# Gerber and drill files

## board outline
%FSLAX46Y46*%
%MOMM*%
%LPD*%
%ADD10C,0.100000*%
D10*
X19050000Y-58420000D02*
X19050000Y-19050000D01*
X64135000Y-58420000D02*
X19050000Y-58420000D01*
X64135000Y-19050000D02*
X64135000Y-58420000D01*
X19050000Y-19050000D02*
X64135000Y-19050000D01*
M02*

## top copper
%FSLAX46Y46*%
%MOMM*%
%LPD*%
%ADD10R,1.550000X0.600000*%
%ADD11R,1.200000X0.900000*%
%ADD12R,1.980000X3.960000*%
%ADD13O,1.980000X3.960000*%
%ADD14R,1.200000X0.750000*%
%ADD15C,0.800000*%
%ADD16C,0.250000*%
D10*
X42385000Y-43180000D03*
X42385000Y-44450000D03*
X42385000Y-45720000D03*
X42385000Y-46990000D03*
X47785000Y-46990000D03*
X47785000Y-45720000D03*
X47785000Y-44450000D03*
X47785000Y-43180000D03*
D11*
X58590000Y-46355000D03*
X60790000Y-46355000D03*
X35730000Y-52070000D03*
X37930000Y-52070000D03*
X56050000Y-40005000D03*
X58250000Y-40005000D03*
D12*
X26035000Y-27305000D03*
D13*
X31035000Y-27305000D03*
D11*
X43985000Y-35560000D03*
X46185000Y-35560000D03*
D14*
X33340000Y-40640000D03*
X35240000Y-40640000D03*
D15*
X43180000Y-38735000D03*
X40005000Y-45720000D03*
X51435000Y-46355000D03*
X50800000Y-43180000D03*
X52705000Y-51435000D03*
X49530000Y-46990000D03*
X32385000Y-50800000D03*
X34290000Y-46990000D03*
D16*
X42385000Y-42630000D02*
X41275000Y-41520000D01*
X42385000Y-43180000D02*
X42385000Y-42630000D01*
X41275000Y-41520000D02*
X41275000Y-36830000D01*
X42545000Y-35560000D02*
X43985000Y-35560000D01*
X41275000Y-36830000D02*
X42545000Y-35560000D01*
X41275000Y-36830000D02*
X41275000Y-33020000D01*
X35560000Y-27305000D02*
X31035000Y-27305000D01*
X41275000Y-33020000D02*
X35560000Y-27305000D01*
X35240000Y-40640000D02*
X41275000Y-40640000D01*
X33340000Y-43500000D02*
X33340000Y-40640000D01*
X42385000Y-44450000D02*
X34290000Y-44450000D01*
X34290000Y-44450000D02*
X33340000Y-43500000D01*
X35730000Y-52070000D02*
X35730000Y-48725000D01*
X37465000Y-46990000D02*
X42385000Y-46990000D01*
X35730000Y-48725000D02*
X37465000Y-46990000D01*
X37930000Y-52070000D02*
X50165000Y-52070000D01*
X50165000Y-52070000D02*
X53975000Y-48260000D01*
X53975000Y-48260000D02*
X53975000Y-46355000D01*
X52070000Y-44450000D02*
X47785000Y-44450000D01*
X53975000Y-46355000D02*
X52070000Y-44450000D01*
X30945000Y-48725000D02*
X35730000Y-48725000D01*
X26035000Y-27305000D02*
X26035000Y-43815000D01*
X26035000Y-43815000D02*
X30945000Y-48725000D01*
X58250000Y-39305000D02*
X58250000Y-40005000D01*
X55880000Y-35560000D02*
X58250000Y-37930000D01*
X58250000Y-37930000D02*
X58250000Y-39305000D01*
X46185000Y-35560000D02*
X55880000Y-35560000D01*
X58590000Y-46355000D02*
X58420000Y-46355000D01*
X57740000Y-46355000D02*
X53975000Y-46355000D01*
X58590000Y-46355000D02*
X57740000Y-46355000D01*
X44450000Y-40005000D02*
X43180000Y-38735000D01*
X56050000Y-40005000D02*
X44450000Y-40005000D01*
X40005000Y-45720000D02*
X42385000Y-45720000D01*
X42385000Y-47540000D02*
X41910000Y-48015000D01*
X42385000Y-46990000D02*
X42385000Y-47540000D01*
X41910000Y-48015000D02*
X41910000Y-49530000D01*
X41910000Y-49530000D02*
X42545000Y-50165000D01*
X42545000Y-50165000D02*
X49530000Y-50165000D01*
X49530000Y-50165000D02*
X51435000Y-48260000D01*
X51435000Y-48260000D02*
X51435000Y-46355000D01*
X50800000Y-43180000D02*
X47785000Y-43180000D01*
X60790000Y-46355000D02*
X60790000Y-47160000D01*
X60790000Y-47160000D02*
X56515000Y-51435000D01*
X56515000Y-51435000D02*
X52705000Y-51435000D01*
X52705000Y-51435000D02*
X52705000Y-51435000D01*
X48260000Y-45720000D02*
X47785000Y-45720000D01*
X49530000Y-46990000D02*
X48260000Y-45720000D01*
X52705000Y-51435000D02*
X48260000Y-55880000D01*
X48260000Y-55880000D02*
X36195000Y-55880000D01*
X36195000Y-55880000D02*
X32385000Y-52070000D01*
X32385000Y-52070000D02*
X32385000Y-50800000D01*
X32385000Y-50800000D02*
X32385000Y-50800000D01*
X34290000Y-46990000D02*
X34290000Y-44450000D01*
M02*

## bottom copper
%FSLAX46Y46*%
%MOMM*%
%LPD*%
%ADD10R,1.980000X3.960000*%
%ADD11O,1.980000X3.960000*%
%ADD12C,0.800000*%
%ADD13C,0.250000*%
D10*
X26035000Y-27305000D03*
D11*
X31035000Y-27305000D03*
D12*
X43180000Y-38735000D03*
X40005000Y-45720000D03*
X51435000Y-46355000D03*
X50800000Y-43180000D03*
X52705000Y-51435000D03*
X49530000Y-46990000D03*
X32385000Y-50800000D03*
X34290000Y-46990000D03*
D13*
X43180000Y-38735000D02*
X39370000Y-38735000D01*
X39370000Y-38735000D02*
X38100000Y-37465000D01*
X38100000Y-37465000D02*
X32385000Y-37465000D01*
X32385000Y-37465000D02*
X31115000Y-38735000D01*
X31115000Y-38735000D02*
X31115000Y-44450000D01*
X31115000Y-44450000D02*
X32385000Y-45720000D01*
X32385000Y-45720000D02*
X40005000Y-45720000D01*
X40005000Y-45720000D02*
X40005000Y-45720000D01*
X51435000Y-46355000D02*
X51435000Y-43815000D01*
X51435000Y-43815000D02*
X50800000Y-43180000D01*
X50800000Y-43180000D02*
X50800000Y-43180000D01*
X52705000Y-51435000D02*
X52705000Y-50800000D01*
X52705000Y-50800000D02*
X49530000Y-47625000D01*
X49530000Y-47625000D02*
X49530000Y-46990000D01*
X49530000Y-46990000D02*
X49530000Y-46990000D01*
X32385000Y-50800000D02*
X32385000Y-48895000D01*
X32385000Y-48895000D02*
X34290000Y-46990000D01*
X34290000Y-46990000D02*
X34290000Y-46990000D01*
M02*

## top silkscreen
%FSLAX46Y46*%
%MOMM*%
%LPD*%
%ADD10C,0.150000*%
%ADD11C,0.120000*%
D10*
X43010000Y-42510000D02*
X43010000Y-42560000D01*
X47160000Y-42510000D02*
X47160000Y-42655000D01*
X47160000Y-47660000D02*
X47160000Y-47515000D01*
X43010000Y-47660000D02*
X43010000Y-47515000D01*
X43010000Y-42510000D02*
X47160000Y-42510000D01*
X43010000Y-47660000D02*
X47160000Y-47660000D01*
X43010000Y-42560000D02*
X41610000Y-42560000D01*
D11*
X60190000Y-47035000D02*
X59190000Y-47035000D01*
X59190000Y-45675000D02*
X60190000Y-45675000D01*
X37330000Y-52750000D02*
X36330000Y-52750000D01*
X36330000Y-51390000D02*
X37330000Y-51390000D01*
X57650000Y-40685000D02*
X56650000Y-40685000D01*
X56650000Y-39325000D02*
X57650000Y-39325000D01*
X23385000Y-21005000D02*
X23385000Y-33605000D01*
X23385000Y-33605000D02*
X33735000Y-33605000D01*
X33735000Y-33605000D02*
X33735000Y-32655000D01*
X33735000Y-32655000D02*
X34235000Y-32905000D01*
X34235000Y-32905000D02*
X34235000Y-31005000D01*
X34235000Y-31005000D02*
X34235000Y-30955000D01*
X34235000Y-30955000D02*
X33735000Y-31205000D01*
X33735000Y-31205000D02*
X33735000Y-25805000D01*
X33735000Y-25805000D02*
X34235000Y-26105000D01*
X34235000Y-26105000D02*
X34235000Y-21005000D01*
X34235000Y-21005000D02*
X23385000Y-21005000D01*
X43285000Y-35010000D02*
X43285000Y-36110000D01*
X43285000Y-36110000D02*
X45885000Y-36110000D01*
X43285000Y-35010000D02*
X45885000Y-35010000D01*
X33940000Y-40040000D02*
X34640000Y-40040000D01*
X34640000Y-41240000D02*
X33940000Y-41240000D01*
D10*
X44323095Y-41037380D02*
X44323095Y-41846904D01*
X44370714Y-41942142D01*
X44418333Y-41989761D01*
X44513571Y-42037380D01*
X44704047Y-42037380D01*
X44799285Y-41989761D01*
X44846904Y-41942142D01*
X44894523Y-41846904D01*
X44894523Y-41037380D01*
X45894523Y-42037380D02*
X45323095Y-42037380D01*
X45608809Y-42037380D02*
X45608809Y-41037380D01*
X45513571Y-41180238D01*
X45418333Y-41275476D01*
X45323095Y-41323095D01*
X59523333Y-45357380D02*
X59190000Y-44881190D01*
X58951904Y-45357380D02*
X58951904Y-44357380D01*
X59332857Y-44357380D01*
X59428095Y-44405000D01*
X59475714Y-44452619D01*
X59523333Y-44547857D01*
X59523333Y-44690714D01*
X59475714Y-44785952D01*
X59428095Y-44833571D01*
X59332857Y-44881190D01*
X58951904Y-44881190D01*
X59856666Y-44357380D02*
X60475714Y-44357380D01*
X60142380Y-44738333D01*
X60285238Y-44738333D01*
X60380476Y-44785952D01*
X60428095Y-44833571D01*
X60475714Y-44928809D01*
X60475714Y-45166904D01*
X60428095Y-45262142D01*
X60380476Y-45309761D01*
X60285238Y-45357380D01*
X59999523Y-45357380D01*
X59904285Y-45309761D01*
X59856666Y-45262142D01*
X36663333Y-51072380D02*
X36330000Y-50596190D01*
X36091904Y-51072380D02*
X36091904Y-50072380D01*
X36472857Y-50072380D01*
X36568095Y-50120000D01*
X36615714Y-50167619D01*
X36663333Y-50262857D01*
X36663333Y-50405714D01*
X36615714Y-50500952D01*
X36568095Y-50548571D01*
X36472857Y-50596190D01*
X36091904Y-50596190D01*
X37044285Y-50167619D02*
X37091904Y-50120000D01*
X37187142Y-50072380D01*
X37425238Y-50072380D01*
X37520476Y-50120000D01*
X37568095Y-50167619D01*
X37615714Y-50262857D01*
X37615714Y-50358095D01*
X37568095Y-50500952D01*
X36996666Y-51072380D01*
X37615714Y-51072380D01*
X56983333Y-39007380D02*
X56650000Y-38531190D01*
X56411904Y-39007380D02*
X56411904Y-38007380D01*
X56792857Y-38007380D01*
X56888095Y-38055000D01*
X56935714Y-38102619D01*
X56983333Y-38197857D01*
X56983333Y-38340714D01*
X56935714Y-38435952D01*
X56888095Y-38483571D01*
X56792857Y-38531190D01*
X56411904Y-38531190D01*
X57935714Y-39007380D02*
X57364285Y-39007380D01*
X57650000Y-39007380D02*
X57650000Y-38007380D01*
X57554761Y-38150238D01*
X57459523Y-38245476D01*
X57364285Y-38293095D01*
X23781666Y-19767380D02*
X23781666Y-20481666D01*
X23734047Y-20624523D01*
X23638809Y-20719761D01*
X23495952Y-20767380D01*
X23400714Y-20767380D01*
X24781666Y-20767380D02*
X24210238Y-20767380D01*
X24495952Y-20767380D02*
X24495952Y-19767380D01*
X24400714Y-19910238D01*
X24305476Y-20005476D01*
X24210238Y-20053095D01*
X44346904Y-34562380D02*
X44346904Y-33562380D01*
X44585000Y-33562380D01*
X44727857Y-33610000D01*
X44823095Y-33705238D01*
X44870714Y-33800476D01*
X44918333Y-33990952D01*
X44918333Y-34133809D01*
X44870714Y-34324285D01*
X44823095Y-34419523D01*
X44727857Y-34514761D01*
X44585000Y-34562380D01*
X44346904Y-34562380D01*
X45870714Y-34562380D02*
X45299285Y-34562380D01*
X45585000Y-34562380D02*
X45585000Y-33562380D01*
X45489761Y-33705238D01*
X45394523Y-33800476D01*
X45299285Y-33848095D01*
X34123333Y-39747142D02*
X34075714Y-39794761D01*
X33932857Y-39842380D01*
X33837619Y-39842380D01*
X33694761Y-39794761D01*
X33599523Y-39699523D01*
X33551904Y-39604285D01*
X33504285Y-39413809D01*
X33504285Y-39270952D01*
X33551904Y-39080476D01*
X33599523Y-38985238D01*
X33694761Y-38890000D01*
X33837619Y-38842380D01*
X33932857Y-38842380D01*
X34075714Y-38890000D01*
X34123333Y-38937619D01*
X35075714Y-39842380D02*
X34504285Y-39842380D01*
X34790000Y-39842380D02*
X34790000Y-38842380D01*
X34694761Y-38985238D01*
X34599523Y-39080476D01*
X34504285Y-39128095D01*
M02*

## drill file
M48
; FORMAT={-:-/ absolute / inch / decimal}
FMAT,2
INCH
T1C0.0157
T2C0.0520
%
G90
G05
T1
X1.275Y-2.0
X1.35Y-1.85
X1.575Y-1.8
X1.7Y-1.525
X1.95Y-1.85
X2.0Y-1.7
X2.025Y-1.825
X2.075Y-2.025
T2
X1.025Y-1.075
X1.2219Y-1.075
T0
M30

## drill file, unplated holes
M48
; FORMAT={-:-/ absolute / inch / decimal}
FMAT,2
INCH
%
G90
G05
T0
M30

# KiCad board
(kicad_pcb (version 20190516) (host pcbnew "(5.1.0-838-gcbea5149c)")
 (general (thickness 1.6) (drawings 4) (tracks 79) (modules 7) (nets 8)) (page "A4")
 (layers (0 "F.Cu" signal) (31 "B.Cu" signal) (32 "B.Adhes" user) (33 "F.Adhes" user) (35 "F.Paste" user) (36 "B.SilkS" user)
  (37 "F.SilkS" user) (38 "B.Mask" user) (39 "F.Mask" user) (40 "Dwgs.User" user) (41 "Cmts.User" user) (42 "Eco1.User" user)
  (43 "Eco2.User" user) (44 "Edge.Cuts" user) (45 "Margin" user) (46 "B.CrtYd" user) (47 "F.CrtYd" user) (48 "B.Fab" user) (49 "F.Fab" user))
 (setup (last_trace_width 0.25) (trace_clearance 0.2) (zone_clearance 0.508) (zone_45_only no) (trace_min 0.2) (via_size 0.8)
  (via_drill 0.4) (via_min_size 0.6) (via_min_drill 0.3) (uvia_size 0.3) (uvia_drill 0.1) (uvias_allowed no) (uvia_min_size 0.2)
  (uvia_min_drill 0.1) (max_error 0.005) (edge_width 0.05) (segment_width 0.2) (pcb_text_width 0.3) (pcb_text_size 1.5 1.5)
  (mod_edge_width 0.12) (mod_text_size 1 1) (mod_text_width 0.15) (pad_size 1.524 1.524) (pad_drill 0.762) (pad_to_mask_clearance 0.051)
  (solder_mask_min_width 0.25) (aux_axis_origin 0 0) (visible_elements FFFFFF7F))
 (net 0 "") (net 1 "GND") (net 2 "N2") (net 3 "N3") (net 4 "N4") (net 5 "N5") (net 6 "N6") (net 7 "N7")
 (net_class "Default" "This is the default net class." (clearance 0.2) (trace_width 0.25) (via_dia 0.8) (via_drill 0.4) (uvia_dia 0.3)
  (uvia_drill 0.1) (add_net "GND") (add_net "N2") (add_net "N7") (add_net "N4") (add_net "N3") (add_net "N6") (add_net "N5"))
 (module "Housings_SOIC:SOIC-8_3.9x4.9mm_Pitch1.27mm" (layer "F.Cu") (at 45.085 45.085)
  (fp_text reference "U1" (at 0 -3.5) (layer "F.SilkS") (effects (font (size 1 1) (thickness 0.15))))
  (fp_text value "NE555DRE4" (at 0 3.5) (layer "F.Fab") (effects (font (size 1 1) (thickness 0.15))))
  (fp_line (start -2.075 -2.575) (end -2.075 -2.525) (layer "F.SilkS") (width 0.15))
  (fp_line (start 2.075 -2.575) (end 2.075 -2.43) (layer "F.SilkS") (width 0.15))
  (fp_line (start 2.075 2.575) (end 2.075 2.43) (layer "F.SilkS") (width 0.15))
  (fp_line (start -2.075 2.575) (end -2.075 2.43) (layer "F.SilkS") (width 0.15))
  (fp_line (start -2.075 -2.575) (end 2.075 -2.575) (layer "F.SilkS") (width 0.15))
  (fp_line (start -2.075 2.575) (end 2.075 2.575) (layer "F.SilkS") (width 0.15))
  (fp_line (start -2.075 -2.525) (end -3.475 -2.525) (layer "F.SilkS") (width 0.15))
  (pad "1" smd rect (at -2.7 -1.905) (size 1.55 0.6) (layers "F.Cu" "F.Paste" "F.Mask") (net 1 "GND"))
  (pad "2" smd rect (at -2.7 -0.635) (size 1.55 0.6) (layers "F.Cu" "F.Paste" "F.Mask") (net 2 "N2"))
  (pad "3" smd rect (at -2.7 0.635) (size 1.55 0.6) (layers "F.Cu" "F.Paste" "F.Mask") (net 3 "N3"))
  (pad "4" smd rect (at -2.7 1.905) (size 1.55 0.6) (layers "F.Cu" "F.Paste" "F.Mask") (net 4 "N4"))
  (pad "5" smd rect (at 2.7 1.905) (size 1.55 0.6) (layers "F.Cu" "F.Paste" "F.Mask") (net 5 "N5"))
  (pad "6" smd rect (at 2.7 0.635) (size 1.55 0.6) (layers "F.Cu" "F.Paste" "F.Mask") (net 2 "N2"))
  (pad "7" smd rect (at 2.7 -0.635) (size 1.55 0.6) (layers "F.Cu" "F.Paste" "F.Mask") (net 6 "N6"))
  (pad "8" smd rect (at 2.7 -1.905) (size 1.55 0.6) (layers "F.Cu" "F.Paste" "F.Mask") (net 4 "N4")))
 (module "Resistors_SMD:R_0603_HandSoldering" (layer "F.Cu") (at 59.69 46.355)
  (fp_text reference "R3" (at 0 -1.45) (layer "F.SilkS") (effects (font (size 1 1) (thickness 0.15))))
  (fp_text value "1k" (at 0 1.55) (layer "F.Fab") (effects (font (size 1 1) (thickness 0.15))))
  (fp_line (start 0.5 0.68) (end -0.5 0.68) (layer "F.SilkS") (width 0.12))
  (fp_line (start -0.5 -0.68) (end 0.5 -0.68) (layer "F.SilkS") (width 0.12))
  (pad "1" smd rect (at -1.1 0) (size 1.2 0.9) (layers "F.Cu" "F.Paste" "F.Mask") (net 6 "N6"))
  (pad "2" smd rect (at 1.1 0) (size 1.2 0.9) (layers "F.Cu" "F.Paste" "F.Mask") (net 2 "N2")))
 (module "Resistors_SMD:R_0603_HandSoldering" (layer "F.Cu") (at 36.83 52.07)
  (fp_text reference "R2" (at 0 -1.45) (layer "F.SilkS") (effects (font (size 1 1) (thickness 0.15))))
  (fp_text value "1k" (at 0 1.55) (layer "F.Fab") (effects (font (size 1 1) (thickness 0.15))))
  (fp_line (start 0.5 0.68) (end -0.5 0.68) (layer "F.SilkS") (width 0.12))
  (fp_line (start -0.5 -0.68) (end 0.5 -0.68) (layer "F.SilkS") (width 0.12))
  (pad "1" smd rect (at -1.1 0) (size 1.2 0.9) (layers "F.Cu" "F.Paste" "F.Mask") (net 4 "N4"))
  (pad "2" smd rect (at 1.1 0) (size 1.2 0.9) (layers "F.Cu" "F.Paste" "F.Mask") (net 6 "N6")))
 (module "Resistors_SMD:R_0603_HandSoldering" (layer "F.Cu") (at 57.15 40.005)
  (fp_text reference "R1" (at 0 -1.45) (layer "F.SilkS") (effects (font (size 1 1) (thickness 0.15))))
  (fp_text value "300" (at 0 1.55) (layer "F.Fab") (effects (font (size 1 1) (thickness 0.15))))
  (fp_line (start 0.5 0.68) (end -0.5 0.68) (layer "F.SilkS") (width 0.12))
  (fp_line (start -0.5 -0.68) (end 0.5 -0.68) (layer "F.SilkS") (width 0.12))
  (pad "1" smd rect (at -1.1 0) (size 1.2 0.9) (layers "F.Cu" "F.Paste" "F.Mask") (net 3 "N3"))
  (pad "2" smd rect (at 1.1 0) (size 1.2 0.9) (layers "F.Cu" "F.Paste" "F.Mask") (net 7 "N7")))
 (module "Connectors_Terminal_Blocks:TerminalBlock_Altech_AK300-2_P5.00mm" (layer "F.Cu") (at 26.035 27.305)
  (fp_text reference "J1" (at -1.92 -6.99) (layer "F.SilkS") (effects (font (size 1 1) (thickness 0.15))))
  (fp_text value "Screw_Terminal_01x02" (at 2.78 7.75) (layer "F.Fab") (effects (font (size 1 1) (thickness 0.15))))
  (fp_line (start -2.65 -6.3) (end -2.65 6.3) (layer "F.SilkS") (width 0.12))
  (fp_line (start -2.65 6.3) (end 7.7 6.3) (layer "F.SilkS") (width 0.12))
  (fp_line (start 7.7 6.3) (end 7.7 5.35) (layer "F.SilkS") (width 0.12))
  (fp_line (start 7.7 5.35) (end 8.2 5.6) (layer "F.SilkS") (width 0.12))
  (fp_line (start 8.2 5.6) (end 8.2 3.7) (layer "F.SilkS") (width 0.12))
  (fp_line (start 8.2 3.7) (end 8.2 3.65) (layer "F.SilkS") (width 0.12))
  (fp_line (start 8.2 3.65) (end 7.7 3.9) (layer "F.SilkS") (width 0.12))
  (fp_line (start 7.7 3.9) (end 7.7 -1.5) (layer "F.SilkS") (width 0.12))
  (fp_line (start 7.7 -1.5) (end 8.2 -1.2) (layer "F.SilkS") (width 0.12))
  (fp_line (start 8.2 -1.2) (end 8.2 -6.3) (layer "F.SilkS") (width 0.12))
  (fp_line (start 8.2 -6.3) (end -2.65 -6.3) (layer "F.SilkS") (width 0.12))
  (pad "1" thru_hole rect (at 0 0) (size 1.98 3.96) (drill 1.32) (layers *.Cu *.Mask) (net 4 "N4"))
  (pad "2" thru_hole oval (at 5 0) (size 1.98 3.96) (drill 1.32) (layers *.Cu *.Mask) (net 1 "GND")))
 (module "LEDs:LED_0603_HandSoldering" (layer "F.Cu") (at 45.085 35.56)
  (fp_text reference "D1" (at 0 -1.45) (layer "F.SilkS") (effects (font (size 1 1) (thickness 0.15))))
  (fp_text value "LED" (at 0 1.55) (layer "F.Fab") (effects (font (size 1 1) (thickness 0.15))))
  (fp_line (start -1.8 -0.55) (end -1.8 0.55) (layer "F.SilkS") (width 0.12))
  (fp_line (start -1.8 0.55) (end 0.8 0.55) (layer "F.SilkS") (width 0.12))
  (fp_line (start -1.8 -0.55) (end 0.8 -0.55) (layer "F.SilkS") (width 0.12))
  (pad "1" smd rect (at -1.1 0) (size 1.2 0.9) (layers "F.Cu" "F.Paste" "F.Mask") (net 1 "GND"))
  (pad "2" smd rect (at 1.1 0) (size 1.2 0.9) (layers "F.Cu" "F.Paste" "F.Mask") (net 7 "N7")))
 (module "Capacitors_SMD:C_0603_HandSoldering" (layer "F.Cu") (at 34.29 40.64)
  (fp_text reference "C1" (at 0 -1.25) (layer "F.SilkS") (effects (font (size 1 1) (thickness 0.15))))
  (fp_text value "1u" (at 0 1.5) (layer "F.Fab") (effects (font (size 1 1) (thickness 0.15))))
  (fp_line (start -0.35 -0.6) (end 0.35 -0.6) (layer "F.SilkS") (width 0.12))
  (fp_line (start 0.35 0.6) (end -0.35 0.6) (layer "F.SilkS") (width 0.12))
  (pad "1" smd rect (at -0.95 0) (size 1.2 0.75) (layers "F.Cu" "F.Paste" "F.Mask") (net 2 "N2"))
  (pad "2" smd rect (at 0.95 0) (size 1.2 0.75) (layers "F.Cu" "F.Paste" "F.Mask") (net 1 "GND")))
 (gr_line (start 19.05 58.42) (end 19.05 19.05) (layer "Edge.Cuts") (width 0.1))
 (gr_line (start 64.135 58.42) (end 19.05 58.42) (layer "Edge.Cuts") (width 0.1))
 (gr_line (start 64.135 19.05) (end 64.135 58.42) (layer "Edge.Cuts") (width 0.1))
 (gr_line (start 19.05 19.05) (end 64.135 19.05) (layer "Edge.Cuts") (width 0.1))
 (segment (start 42.385 42.63) (end 41.275 41.52) (width 0.25) (layer "F.Cu") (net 1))
 (segment (start 42.385 43.18) (end 42.385 42.63) (width 0.25) (layer "F.Cu") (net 1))
 (segment (start 41.275 41.52) (end 41.275 36.83) (width 0.25) (layer "F.Cu") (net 1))
 (segment (start 42.545 35.56) (end 43.985 35.56) (width 0.25) (layer "F.Cu") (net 1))
 (segment (start 41.275 36.83) (end 42.545 35.56) (width 0.25) (layer "F.Cu") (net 1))
 (segment (start 41.275 36.83) (end 41.275 33.02) (width 0.25) (layer "F.Cu") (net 1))
 (segment (start 35.56 27.305) (end 31.035 27.305) (width 0.25) (layer "F.Cu") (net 1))
 (segment (start 41.275 33.02) (end 35.56 27.305) (width 0.25) (layer "F.Cu") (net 1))
 (segment (start 35.24 40.64) (end 41.275 40.64) (width 0.25) (layer "F.Cu") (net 1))
 (segment (start 33.34 43.5) (end 33.34 40.64) (width 0.25) (layer "F.Cu") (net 2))
 (segment (start 42.385 44.45) (end 34.29 44.45) (width 0.25) (layer "F.Cu") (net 2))
 (segment (start 34.29 44.45) (end 33.34 43.5) (width 0.25) (layer "F.Cu") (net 2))
 (segment (start 35.73 52.07) (end 35.73 48.725) (width 0.25) (layer "F.Cu") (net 4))
 (segment (start 37.465 46.99) (end 42.385 46.99) (width 0.25) (layer "F.Cu") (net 4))
 (segment (start 35.73 48.725) (end 37.465 46.99) (width 0.25) (layer "F.Cu") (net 4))
 (segment (start 37.93 52.07) (end 50.165 52.07) (width 0.25) (layer "F.Cu") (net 6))
 (segment (start 50.165 52.07) (end 53.975 48.26) (width 0.25) (layer "F.Cu") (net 6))
 (segment (start 53.975 48.26) (end 53.975 46.355) (width 0.25) (layer "F.Cu") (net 6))
 (segment (start 52.07 44.45) (end 47.785 44.45) (width 0.25) (layer "F.Cu") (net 6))
 (segment (start 53.975 46.355) (end 52.07 44.45) (width 0.25) (layer "F.Cu") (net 6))
 (segment (start 30.945 48.725) (end 35.73 48.725) (width 0.25) (layer "F.Cu") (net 4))
 (segment (start 26.035 27.305) (end 26.035 43.815) (width 0.25) (layer "F.Cu") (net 4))
 (segment (start 26.035 43.815) (end 30.945 48.725) (width 0.25) (layer "F.Cu") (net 4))
 (segment (start 58.25 39.305) (end 58.25 40.005) (width 0.25) (layer "F.Cu") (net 7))
 (segment (start 55.88 35.56) (end 58.25 37.93) (width 0.25) (layer "F.Cu") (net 7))
 (segment (start 58.25 37.93) (end 58.25 39.305) (width 0.25) (layer "F.Cu") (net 7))
 (segment (start 46.185 35.56) (end 55.88 35.56) (width 0.25) (layer "F.Cu") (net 7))
 (segment (start 58.59 46.355) (end 58.42 46.355) (width 0.25) (layer "F.Cu") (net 6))
 (segment (start 57.74 46.355) (end 53.975 46.355) (width 0.25) (layer "F.Cu") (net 6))
 (segment (start 58.59 46.355) (end 57.74 46.355) (width 0.25) (layer "F.Cu") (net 6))
 (via (at 43.18 38.735) (size 0.8) (drill 0.4) (layers "F.Cu" "B.Cu") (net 3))
 (segment (start 44.45 40.005) (end 43.18 38.735) (width 0.25) (layer "F.Cu") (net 3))
 (segment (start 56.05 40.005) (end 44.45 40.005) (width 0.25) (layer "F.Cu") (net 3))
 (segment (start 43.18 38.735) (end 39.37 38.735) (width 0.25) (layer "B.Cu") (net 3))
 (segment (start 39.37 38.735) (end 38.1 37.465) (width 0.25) (layer "B.Cu") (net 3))
 (segment (start 38.1 37.465) (end 32.385 37.465) (width 0.25) (layer "B.Cu") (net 3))
 (segment (start 32.385 37.465) (end 31.115 38.735) (width 0.25) (layer "B.Cu") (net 3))
 (segment (start 31.115 38.735) (end 31.115 44.45) (width 0.25) (layer "B.Cu") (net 3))
 (segment (start 31.115 44.45) (end 32.385 45.72) (width 0.25) (layer "B.Cu") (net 3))
 (segment (start 32.385 45.72) (end 40.005 45.72) (width 0.25) (layer "B.Cu") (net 3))
 (segment (start 40.005 45.72) (end 40.005 45.72) (width 0.25) (layer "B.Cu") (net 3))
 (via (at 40.005 45.72) (size 0.8) (drill 0.4) (layers "F.Cu" "B.Cu") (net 3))
 (segment (start 40.005 45.72) (end 42.385 45.72) (width 0.25) (layer "F.Cu") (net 3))
 (segment (start 42.385 47.54) (end 41.91 48.015) (width 0.25) (layer "F.Cu") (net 4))
 (segment (start 42.385 46.99) (end 42.385 47.54) (width 0.25) (layer "F.Cu") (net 4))
 (segment (start 41.91 48.015) (end 41.91 49.53) (width 0.25) (layer "F.Cu") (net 4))
 (segment (start 41.91 49.53) (end 42.545 50.165) (width 0.25) (layer "F.Cu") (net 4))
 (segment (start 42.545 50.165) (end 49.53 50.165) (width 0.25) (layer "F.Cu") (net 4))
 (segment (start 49.53 50.165) (end 51.435 48.26) (width 0.25) (layer "F.Cu") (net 4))
 (segment (start 51.435 48.26) (end 51.435 46.355) (width 0.25) (layer "F.Cu") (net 4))
 (via (at 51.435 46.355) (size 0.8) (drill 0.4) (layers "F.Cu" "B.Cu") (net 4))
 (segment (start 51.435 46.355) (end 51.435 43.815) (width 0.25) (layer "B.Cu") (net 4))
 (segment (start 51.435 43.815) (end 50.8 43.18) (width 0.25) (layer "B.Cu") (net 4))
 (segment (start 50.8 43.18) (end 50.8 43.18) (width 0.25) (layer "B.Cu") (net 4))
 (via (at 50.8 43.18) (size 0.8) (drill 0.4) (layers "F.Cu" "B.Cu") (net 4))
 (segment (start 50.8 43.18) (end 47.785 43.18) (width 0.25) (layer "F.Cu") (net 4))
 (segment (start 60.79 46.355) (end 60.79 47.16) (width 0.25) (layer "F.Cu") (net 2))
 (segment (start 60.79 47.16) (end 56.515 51.435) (width 0.25) (layer "F.Cu") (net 2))
 (segment (start 56.515 51.435) (end 52.705 51.435) (width 0.25) (layer "F.Cu") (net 2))
 (segment (start 52.705 51.435) (end 52.705 51.435) (width 0.25) (layer "F.Cu") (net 2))
 (via (at 52.705 51.435) (size 0.8) (drill 0.4) (layers "F.Cu" "B.Cu") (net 2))
 (segment (start 52.705 51.435) (end 52.705 50.8) (width 0.25) (layer "B.Cu") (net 2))
 (segment (start 52.705 50.8) (end 49.53 47.625) (width 0.25) (layer "B.Cu") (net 2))
 (segment (start 49.53 47.625) (end 49.53 46.99) (width 0.25) (layer "B.Cu") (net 2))
 (segment (start 49.53 46.99) (end 49.53 46.99) (width 0.25) (layer "B.Cu") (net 2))
 (via (at 49.53 46.99) (size 0.8) (drill 0.4) (layers "F.Cu" "B.Cu") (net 2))
 (segment (start 48.26 45.72) (end 47.785 45.72) (width 0.25) (layer "F.Cu") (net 2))
 (segment (start 49.53 46.99) (end 48.26 45.72) (width 0.25) (layer "F.Cu") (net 2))
 (segment (start 52.705 51.435) (end 48.26 55.88) (width 0.25) (layer "F.Cu") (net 2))
 (segment (start 48.26 55.88) (end 36.195 55.88) (width 0.25) (layer "F.Cu") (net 2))
 (segment (start 36.195 55.88) (end 32.385 52.07) (width 0.25) (layer "F.Cu") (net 2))
 (segment (start 32.385 52.07) (end 32.385 50.8) (width 0.25) (layer "F.Cu") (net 2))
 (segment (start 32.385 50.8) (end 32.385 50.8) (width 0.25) (layer "F.Cu") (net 2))
 (via (at 32.385 50.8) (size 0.8) (drill 0.4) (layers "F.Cu" "B.Cu") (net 2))
 (segment (start 32.385 50.8) (end 32.385 48.895) (width 0.25) (layer "B.Cu") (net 2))
 (segment (start 32.385 48.895) (end 34.29 46.99) (width 0.25) (layer "B.Cu") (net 2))
 (segment (start 34.29 46.99) (end 34.29 46.99) (width 0.25) (layer "B.Cu") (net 2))
 (via (at 34.29 46.99) (size 0.8) (drill 0.4) (layers "F.Cu" "B.Cu") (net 2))
 (segment (start 34.29 46.99) (end 34.29 44.45) (width 0.25) (layer "F.Cu") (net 2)))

